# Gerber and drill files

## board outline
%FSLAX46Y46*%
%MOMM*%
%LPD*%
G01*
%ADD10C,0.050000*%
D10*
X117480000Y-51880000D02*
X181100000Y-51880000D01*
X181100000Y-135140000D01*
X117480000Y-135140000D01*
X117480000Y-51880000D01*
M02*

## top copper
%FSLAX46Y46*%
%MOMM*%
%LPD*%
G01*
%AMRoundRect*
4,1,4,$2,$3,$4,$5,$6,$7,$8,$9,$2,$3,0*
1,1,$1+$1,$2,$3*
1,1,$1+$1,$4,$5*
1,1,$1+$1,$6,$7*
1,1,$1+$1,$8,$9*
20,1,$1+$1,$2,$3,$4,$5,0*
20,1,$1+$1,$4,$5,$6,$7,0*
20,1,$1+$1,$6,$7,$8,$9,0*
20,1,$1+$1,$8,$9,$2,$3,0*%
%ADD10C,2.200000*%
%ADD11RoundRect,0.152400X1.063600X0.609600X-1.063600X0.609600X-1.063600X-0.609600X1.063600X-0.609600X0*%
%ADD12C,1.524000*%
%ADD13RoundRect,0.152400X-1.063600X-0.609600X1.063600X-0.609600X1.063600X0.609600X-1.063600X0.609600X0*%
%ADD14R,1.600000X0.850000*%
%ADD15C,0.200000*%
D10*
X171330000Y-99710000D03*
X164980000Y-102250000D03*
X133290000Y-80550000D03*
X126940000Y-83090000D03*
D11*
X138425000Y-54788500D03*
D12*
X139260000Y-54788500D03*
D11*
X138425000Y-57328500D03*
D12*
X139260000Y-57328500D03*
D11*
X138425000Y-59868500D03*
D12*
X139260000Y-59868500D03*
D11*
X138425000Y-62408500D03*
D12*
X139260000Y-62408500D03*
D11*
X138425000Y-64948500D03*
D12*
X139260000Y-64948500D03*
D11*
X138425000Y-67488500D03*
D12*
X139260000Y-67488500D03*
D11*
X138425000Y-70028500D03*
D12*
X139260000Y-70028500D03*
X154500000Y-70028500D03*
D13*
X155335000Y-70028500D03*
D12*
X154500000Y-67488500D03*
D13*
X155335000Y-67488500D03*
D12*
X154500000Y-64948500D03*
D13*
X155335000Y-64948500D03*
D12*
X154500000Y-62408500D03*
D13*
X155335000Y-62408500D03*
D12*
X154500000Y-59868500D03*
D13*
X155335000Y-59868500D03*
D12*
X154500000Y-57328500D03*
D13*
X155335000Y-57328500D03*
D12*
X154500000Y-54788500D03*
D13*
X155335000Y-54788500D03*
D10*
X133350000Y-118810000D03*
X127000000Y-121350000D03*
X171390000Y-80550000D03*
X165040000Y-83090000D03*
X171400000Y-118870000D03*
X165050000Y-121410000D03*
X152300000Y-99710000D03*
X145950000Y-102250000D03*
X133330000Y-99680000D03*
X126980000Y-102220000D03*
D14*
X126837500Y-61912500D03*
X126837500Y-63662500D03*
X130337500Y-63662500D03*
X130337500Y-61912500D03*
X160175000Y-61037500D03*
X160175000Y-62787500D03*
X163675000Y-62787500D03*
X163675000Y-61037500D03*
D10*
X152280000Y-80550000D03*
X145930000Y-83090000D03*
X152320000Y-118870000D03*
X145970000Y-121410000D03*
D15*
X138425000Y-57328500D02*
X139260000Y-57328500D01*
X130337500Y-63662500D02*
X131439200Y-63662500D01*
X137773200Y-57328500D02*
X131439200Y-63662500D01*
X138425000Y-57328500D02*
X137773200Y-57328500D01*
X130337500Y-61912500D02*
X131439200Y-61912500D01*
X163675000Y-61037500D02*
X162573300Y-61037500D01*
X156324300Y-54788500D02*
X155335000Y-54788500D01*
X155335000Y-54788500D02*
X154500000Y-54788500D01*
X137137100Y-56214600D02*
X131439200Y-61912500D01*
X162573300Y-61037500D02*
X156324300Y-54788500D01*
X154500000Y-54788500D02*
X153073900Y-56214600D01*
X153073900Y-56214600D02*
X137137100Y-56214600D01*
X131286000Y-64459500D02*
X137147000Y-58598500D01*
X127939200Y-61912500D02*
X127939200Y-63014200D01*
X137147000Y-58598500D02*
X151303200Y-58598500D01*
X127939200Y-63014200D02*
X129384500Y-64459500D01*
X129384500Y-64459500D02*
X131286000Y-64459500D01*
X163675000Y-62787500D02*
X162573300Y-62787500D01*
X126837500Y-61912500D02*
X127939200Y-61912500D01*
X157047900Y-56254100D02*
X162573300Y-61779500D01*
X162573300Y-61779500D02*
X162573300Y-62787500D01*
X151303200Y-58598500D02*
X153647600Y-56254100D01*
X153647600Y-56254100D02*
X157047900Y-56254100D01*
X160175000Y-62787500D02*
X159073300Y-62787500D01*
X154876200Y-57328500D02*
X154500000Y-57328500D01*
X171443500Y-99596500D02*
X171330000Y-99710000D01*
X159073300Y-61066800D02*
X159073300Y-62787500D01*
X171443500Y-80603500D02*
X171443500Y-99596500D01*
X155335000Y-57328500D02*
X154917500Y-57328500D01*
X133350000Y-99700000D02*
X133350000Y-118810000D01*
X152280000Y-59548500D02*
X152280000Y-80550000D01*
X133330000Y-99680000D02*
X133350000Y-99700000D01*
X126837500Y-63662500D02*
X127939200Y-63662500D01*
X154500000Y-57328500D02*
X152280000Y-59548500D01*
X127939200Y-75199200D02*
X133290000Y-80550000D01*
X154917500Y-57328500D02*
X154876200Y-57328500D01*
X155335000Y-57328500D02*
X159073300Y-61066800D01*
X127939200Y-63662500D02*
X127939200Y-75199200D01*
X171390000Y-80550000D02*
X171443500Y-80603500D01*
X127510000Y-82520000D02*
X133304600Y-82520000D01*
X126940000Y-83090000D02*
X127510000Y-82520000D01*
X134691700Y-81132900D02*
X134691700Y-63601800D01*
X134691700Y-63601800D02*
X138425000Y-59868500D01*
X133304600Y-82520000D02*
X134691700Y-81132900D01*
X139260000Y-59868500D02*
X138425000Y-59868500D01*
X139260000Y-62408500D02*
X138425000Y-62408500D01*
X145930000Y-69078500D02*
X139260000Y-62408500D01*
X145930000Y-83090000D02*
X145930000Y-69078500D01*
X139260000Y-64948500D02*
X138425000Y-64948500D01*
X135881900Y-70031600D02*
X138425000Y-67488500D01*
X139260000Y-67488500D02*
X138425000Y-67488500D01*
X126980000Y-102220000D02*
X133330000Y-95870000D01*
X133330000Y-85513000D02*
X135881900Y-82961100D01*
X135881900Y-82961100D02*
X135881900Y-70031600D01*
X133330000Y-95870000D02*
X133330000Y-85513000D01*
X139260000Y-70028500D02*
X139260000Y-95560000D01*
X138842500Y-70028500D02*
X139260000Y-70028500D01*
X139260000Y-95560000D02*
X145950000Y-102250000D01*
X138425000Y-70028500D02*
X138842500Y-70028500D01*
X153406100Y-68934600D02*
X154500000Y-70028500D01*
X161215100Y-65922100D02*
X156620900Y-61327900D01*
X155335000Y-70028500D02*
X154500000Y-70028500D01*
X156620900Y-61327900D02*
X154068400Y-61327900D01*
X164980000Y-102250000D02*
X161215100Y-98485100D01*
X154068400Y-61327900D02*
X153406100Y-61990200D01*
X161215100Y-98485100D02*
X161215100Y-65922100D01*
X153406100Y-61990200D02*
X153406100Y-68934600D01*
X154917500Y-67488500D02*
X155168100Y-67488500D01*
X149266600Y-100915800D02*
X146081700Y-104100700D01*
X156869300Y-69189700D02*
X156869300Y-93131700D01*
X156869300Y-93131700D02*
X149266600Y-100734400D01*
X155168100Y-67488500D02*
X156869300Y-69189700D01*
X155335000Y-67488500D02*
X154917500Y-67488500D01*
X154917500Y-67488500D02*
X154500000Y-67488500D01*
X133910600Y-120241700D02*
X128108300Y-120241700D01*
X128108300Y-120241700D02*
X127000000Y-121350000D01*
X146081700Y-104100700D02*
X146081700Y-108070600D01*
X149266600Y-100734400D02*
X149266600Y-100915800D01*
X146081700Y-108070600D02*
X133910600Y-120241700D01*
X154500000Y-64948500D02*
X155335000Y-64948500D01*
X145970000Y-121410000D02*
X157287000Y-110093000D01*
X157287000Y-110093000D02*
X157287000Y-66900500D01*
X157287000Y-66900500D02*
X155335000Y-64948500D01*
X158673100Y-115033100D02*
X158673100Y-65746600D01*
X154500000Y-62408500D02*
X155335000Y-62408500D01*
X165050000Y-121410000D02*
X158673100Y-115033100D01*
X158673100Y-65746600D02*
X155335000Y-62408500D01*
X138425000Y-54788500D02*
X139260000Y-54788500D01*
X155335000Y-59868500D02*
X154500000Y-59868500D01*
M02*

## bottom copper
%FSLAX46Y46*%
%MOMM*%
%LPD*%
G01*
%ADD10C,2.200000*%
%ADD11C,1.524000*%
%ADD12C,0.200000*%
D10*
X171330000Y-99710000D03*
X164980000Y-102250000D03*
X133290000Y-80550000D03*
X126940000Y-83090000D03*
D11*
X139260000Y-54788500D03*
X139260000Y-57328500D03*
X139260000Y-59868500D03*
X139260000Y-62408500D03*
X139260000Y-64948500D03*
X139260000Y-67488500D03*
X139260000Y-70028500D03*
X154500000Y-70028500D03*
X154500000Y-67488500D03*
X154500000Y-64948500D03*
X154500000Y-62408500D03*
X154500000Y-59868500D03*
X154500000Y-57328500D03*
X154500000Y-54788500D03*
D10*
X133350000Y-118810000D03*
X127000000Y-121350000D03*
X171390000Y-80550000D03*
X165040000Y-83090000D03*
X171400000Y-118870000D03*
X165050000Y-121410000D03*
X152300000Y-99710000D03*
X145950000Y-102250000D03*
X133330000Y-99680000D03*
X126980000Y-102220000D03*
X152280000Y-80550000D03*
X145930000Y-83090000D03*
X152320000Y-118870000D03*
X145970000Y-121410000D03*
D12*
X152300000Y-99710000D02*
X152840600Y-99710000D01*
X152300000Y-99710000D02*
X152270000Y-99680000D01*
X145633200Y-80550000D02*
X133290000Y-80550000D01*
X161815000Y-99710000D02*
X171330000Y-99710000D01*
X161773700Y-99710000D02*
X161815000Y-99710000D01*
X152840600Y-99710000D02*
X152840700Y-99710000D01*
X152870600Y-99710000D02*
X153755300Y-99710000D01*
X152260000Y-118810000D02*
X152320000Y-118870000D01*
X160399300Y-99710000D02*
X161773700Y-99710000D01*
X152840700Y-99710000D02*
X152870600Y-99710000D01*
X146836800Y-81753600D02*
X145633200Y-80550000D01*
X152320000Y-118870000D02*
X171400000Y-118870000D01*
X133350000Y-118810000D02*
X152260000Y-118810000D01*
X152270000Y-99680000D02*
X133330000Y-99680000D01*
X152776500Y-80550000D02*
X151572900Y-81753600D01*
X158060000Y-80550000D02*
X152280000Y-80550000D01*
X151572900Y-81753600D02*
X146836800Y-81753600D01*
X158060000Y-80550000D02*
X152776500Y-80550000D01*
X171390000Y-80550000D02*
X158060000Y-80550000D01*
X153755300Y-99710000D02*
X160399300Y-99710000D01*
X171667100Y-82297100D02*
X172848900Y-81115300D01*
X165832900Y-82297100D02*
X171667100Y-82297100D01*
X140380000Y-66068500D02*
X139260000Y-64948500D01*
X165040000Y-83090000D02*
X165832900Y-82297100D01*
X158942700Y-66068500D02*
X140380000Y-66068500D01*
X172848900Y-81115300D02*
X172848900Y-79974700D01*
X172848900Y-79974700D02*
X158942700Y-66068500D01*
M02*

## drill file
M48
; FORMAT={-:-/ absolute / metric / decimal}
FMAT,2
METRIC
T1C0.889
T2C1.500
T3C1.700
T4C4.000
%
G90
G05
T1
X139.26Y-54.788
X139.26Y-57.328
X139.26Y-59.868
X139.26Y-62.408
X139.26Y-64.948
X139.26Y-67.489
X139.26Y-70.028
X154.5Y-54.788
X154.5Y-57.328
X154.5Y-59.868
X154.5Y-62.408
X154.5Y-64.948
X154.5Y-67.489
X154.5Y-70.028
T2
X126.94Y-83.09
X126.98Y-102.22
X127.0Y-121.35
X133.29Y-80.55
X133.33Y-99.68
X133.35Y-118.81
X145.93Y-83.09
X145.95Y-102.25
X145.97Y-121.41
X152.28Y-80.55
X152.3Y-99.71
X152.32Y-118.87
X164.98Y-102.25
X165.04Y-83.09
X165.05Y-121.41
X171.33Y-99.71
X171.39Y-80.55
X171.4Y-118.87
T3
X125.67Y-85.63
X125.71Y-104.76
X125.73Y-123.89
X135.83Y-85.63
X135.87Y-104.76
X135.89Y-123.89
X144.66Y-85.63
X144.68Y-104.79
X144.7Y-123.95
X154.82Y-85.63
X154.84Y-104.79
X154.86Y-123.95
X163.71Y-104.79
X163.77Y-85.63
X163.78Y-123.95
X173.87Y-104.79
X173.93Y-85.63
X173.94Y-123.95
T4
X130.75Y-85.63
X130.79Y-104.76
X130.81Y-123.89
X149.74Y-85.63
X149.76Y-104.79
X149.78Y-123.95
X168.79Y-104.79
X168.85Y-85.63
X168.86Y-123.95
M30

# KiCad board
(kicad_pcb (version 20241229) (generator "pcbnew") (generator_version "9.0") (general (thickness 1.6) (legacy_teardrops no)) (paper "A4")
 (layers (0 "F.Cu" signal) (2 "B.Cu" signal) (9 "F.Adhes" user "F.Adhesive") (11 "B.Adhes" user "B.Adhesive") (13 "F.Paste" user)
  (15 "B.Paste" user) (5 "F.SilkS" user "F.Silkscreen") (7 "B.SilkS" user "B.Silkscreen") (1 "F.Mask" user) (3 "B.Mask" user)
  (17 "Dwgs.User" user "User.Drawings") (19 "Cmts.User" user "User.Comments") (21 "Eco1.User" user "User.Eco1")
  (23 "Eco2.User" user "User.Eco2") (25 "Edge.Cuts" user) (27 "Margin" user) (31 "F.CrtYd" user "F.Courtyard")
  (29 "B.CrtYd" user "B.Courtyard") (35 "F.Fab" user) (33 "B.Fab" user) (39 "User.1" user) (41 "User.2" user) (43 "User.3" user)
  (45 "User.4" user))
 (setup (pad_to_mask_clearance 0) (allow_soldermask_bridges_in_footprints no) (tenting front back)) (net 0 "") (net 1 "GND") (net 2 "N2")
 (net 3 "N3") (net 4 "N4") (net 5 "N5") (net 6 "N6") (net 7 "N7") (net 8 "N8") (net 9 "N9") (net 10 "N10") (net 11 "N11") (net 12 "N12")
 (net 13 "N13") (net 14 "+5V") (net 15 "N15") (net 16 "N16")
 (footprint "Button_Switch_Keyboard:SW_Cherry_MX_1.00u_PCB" (layer "F.Cu") (at 171.33 99.71)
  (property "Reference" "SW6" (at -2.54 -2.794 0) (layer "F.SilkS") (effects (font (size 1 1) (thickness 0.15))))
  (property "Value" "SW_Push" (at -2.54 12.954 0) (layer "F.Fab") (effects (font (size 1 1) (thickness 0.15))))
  (pad "" np_thru_hole circle (at -7.62 5.08) (size 1.7 1.7) (drill 1.7) (layers "*.Cu" "*.Mask"))
  (pad "" np_thru_hole circle (at -2.54 5.08) (size 4 4) (drill 4) (layers "*.Cu" "*.Mask"))
  (pad "" np_thru_hole circle (at 2.54 5.08) (size 1.7 1.7) (drill 1.7) (layers "*.Cu" "*.Mask"))
  (pad "1" thru_hole circle (at 0 0) (size 2.2 2.2) (drill 1.5) (layers "*.Cu" "*.Mask") (remove_unused_layers no) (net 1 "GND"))
  (pad "2" thru_hole circle (at -6.35 2.54) (size 2.2 2.2) (drill 1.5) (layers "*.Cu" "*.Mask") (remove_unused_layers no) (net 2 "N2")))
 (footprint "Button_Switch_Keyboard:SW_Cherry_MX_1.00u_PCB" (layer "F.Cu") (at 133.29 80.55)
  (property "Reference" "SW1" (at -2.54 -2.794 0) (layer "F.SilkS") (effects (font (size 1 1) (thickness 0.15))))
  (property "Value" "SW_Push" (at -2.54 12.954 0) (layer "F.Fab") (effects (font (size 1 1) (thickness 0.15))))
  (pad "" np_thru_hole circle (at -7.62 5.08) (size 1.7 1.7) (drill 1.7) (layers "*.Cu" "*.Mask"))
  (pad "" np_thru_hole circle (at -2.54 5.08) (size 4 4) (drill 4) (layers "*.Cu" "*.Mask"))
  (pad "" np_thru_hole circle (at 2.54 5.08) (size 1.7 1.7) (drill 1.7) (layers "*.Cu" "*.Mask"))
  (pad "1" thru_hole circle (at 0 0) (size 2.2 2.2) (drill 1.5) (layers "*.Cu" "*.Mask") (remove_unused_layers no) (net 1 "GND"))
  (pad "2" thru_hole circle (at -6.35 2.54) (size 2.2 2.2) (drill 1.5) (layers "*.Cu" "*.Mask") (remove_unused_layers no) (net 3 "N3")))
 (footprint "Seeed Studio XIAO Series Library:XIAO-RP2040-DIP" (layer "F.Cu") (at 146.88 62.4085)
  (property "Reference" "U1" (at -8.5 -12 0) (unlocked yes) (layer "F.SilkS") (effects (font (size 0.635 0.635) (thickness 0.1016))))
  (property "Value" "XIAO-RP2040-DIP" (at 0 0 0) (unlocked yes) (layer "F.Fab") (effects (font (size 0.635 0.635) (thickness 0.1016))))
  (pad "1" smd roundrect (at -8.455 -7.62 180) (size 2.432 1.524) (layers "F.Cu" "F.Mask") (roundrect_rratio 0.1) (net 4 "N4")
   (thermal_bridge_angle 45))
  (pad "1" thru_hole circle (at -7.62 -7.62 180) (size 1.524 1.524) (drill 0.889) (layers "*.Cu" "*.Mask") (remove_unused_layers no)
   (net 4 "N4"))
  (pad "2" smd roundrect (at -8.455 -5.08 180) (size 2.432 1.524) (layers "F.Cu" "F.Mask") (roundrect_rratio 0.1) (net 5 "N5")
   (thermal_bridge_angle 45))
  (pad "2" thru_hole circle (at -7.62 -5.08 180) (size 1.524 1.524) (drill 0.889) (layers "*.Cu" "*.Mask") (remove_unused_layers no)
   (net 5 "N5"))
  (pad "3" smd roundrect (at -8.455 -2.54 180) (size 2.432 1.524) (layers "F.Cu" "F.Mask") (roundrect_rratio 0.1) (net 3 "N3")
   (thermal_bridge_angle 45))
  (pad "3" thru_hole circle (at -7.62 -2.54 180) (size 1.524 1.524) (drill 0.889) (layers "*.Cu" "*.Mask") (remove_unused_layers no)
   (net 3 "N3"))
  (pad "4" smd roundrect (at -8.455 0 180) (size 2.432 1.524) (layers "F.Cu" "F.Mask") (roundrect_rratio 0.1) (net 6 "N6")
   (thermal_bridge_angle 45))
  (pad "4" thru_hole circle (at -7.62 0 180) (size 1.524 1.524) (drill 0.889) (layers "*.Cu" "*.Mask") (remove_unused_layers no)
   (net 6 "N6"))
  (pad "5" smd roundrect (at -8.455 2.54 180) (size 2.432 1.524) (layers "F.Cu" "F.Mask") (roundrect_rratio 0.1) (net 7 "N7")
   (thermal_bridge_angle 45))
  (pad "5" thru_hole circle (at -7.62 2.54 180) (size 1.524 1.524) (drill 0.889) (layers "*.Cu" "*.Mask") (remove_unused_layers no)
   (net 7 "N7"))
  (pad "6" smd roundrect (at -8.455 5.08 180) (size 2.432 1.524) (layers "F.Cu" "F.Mask") (roundrect_rratio 0.1) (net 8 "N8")
   (thermal_bridge_angle 45))
  (pad "6" thru_hole circle (at -7.62 5.08 180) (size 1.524 1.524) (drill 0.889) (layers "*.Cu" "*.Mask") (remove_unused_layers no)
   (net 8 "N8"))
  (pad "7" smd roundrect (at -8.455 7.62 180) (size 2.432 1.524) (layers "F.Cu" "F.Mask") (roundrect_rratio 0.1) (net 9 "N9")
   (thermal_bridge_angle 45))
  (pad "7" thru_hole circle (at -7.62 7.62 180) (size 1.524 1.524) (drill 0.889) (layers "*.Cu" "*.Mask") (remove_unused_layers no)
   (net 9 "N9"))
  (pad "8" thru_hole circle (at 7.62 7.62) (size 1.524 1.524) (drill 0.889) (layers "*.Cu" "*.Mask") (remove_unused_layers no) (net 2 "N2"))
  (pad "8" smd roundrect (at 8.455 7.62) (size 2.432 1.524) (layers "F.Cu" "F.Mask") (roundrect_rratio 0.1) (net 2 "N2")
   (thermal_bridge_angle 45))
  (pad "9" thru_hole circle (at 7.62 5.08) (size 1.524 1.524) (drill 0.889) (layers "*.Cu" "*.Mask") (remove_unused_layers no)
   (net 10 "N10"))
  (pad "9" smd roundrect (at 8.455 5.08) (size 2.432 1.524) (layers "F.Cu" "F.Mask") (roundrect_rratio 0.1) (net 10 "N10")
   (thermal_bridge_angle 45))
  (pad "10" thru_hole circle (at 7.62 2.54) (size 1.524 1.524) (drill 0.889) (layers "*.Cu" "*.Mask") (remove_unused_layers no)
   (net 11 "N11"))
  (pad "10" smd roundrect (at 8.455 2.54) (size 2.432 1.524) (layers "F.Cu" "F.Mask") (roundrect_rratio 0.1) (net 11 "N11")
   (thermal_bridge_angle 45))
  (pad "11" thru_hole circle (at 7.62 0) (size 1.524 1.524) (drill 0.889) (layers "*.Cu" "*.Mask") (remove_unused_layers no) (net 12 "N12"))
  (pad "11" smd roundrect (at 8.455 0) (size 2.432 1.524) (layers "F.Cu" "F.Mask") (roundrect_rratio 0.1) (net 12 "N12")
   (thermal_bridge_angle 45))
  (pad "12" thru_hole circle (at 7.62 -2.54) (size 1.524 1.524) (drill 0.889) (layers "*.Cu" "*.Mask") (remove_unused_layers no)
   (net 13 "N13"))
  (pad "12" smd roundrect (at 8.455 -2.54) (size 2.432 1.524) (layers "F.Cu" "F.Mask") (roundrect_rratio 0.1) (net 13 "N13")
   (thermal_bridge_angle 45))
  (pad "13" thru_hole circle (at 7.62 -5.08) (size 1.524 1.524) (drill 0.889) (layers "*.Cu" "*.Mask") (remove_unused_layers no)
   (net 1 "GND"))
  (pad "13" smd roundrect (at 8.455 -5.08) (size 2.432 1.524) (layers "F.Cu" "F.Mask") (roundrect_rratio 0.1) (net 1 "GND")
   (thermal_bridge_angle 45))
  (pad "14" thru_hole circle (at 7.62 -7.62) (size 1.524 1.524) (drill 0.889) (layers "*.Cu" "*.Mask") (remove_unused_layers no)
   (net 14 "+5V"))
  (pad "14" smd roundrect (at 8.455 -7.62) (size 2.432 1.524) (layers "F.Cu" "F.Mask") (roundrect_rratio 0.1) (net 14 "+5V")
   (thermal_bridge_angle 45)))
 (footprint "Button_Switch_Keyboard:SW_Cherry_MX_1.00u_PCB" (layer "F.Cu") (at 133.35 118.81)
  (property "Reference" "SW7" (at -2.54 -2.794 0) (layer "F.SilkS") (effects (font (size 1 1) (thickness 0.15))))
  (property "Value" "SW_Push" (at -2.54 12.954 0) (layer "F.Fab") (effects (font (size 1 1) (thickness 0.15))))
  (pad "" np_thru_hole circle (at -7.62 5.08) (size 1.7 1.7) (drill 1.7) (layers "*.Cu" "*.Mask"))
  (pad "" np_thru_hole circle (at -2.54 5.08) (size 4 4) (drill 4) (layers "*.Cu" "*.Mask"))
  (pad "" np_thru_hole circle (at 2.54 5.08) (size 1.7 1.7) (drill 1.7) (layers "*.Cu" "*.Mask"))
  (pad "1" thru_hole circle (at 0 0) (size 2.2 2.2) (drill 1.5) (layers "*.Cu" "*.Mask") (remove_unused_layers no) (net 1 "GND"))
  (pad "2" thru_hole circle (at -6.35 2.54) (size 2.2 2.2) (drill 1.5) (layers "*.Cu" "*.Mask") (remove_unused_layers no) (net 10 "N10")))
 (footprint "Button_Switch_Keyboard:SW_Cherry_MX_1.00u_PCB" (layer "F.Cu") (at 171.39 80.55)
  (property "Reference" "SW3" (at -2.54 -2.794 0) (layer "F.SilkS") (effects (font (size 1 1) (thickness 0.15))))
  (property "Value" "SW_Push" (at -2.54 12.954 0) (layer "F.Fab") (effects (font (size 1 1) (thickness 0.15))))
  (pad "" np_thru_hole circle (at -7.62 5.08) (size 1.7 1.7) (drill 1.7) (layers "*.Cu" "*.Mask"))
  (pad "" np_thru_hole circle (at -2.54 5.08) (size 4 4) (drill 4) (layers "*.Cu" "*.Mask"))
  (pad "" np_thru_hole circle (at 2.54 5.08) (size 1.7 1.7) (drill 1.7) (layers "*.Cu" "*.Mask"))
  (pad "1" thru_hole circle (at 0 0) (size 2.2 2.2) (drill 1.5) (layers "*.Cu" "*.Mask") (remove_unused_layers no) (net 1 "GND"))
  (pad "2" thru_hole circle (at -6.35 2.54) (size 2.2 2.2) (drill 1.5) (layers "*.Cu" "*.Mask") (remove_unused_layers no) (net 7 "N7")))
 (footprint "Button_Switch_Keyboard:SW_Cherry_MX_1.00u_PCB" (layer "F.Cu") (at 171.4 118.87)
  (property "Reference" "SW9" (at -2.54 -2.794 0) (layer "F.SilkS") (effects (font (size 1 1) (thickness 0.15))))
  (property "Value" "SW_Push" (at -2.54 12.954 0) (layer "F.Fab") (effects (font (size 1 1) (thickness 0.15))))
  (pad "" np_thru_hole circle (at -7.62 5.08) (size 1.7 1.7) (drill 1.7) (layers "*.Cu" "*.Mask"))
  (pad "" np_thru_hole circle (at -2.54 5.08) (size 4 4) (drill 4) (layers "*.Cu" "*.Mask"))
  (pad "" np_thru_hole circle (at 2.54 5.08) (size 1.7 1.7) (drill 1.7) (layers "*.Cu" "*.Mask"))
  (pad "1" thru_hole circle (at 0 0) (size 2.2 2.2) (drill 1.5) (layers "*.Cu" "*.Mask") (remove_unused_layers no) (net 1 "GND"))
  (pad "2" thru_hole circle (at -6.35 2.54) (size 2.2 2.2) (drill 1.5) (layers "*.Cu" "*.Mask") (remove_unused_layers no) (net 12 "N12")))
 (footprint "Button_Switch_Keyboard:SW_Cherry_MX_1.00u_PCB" (layer "F.Cu") (at 152.3 99.71)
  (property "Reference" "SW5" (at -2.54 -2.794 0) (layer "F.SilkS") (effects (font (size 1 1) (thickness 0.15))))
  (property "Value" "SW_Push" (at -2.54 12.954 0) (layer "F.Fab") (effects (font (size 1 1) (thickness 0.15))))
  (pad "" np_thru_hole circle (at -7.62 5.08) (size 1.7 1.7) (drill 1.7) (layers "*.Cu" "*.Mask"))
  (pad "" np_thru_hole circle (at -2.54 5.08) (size 4 4) (drill 4) (layers "*.Cu" "*.Mask"))
  (pad "" np_thru_hole circle (at 2.54 5.08) (size 1.7 1.7) (drill 1.7) (layers "*.Cu" "*.Mask"))
  (pad "1" thru_hole circle (at 0 0) (size 2.2 2.2) (drill 1.5) (layers "*.Cu" "*.Mask") (remove_unused_layers no) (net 1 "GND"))
  (pad "2" thru_hole circle (at -6.35 2.54) (size 2.2 2.2) (drill 1.5) (layers "*.Cu" "*.Mask") (remove_unused_layers no) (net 9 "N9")))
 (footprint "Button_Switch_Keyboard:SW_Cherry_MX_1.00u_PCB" (layer "F.Cu") (at 133.33 99.68)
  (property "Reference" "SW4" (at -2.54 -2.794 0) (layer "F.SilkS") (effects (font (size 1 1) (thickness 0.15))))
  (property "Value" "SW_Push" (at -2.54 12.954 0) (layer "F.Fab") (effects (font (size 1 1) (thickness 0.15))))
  (pad "" np_thru_hole circle (at -7.62 5.08) (size 1.7 1.7) (drill 1.7) (layers "*.Cu" "*.Mask"))
  (pad "" np_thru_hole circle (at -2.54 5.08) (size 4 4) (drill 4) (layers "*.Cu" "*.Mask"))
  (pad "" np_thru_hole circle (at 2.54 5.08) (size 1.7 1.7) (drill 1.7) (layers "*.Cu" "*.Mask"))
  (pad "1" thru_hole circle (at 0 0) (size 2.2 2.2) (drill 1.5) (layers "*.Cu" "*.Mask") (remove_unused_layers no) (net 1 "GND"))
  (pad "2" thru_hole circle (at -6.35 2.54) (size 2.2 2.2) (drill 1.5) (layers "*.Cu" "*.Mask") (remove_unused_layers no) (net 8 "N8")))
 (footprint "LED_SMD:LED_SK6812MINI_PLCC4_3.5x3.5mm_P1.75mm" (layer "F.Cu") (at 128.5875 62.7875)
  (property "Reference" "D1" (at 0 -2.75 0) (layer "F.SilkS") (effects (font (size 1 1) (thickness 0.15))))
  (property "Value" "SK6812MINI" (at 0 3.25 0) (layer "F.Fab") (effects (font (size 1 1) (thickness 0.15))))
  (pad "1" smd rect (at -1.75 -0.875) (size 1.6 0.85) (layers "F.Cu" "F.Mask" "F.Paste") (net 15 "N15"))
  (pad "2" smd rect (at -1.75 0.875) (size 1.6 0.85) (layers "F.Cu" "F.Mask" "F.Paste") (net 1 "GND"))
  (pad "3" smd rect (at 1.75 0.875) (size 1.6 0.85) (layers "F.Cu" "F.Mask" "F.Paste") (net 5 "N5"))
  (pad "4" smd rect (at 1.75 -0.875) (size 1.6 0.85) (layers "F.Cu" "F.Mask" "F.Paste") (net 14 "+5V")))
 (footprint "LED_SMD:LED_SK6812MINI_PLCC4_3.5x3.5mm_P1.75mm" (layer "F.Cu") (at 161.925 61.9125)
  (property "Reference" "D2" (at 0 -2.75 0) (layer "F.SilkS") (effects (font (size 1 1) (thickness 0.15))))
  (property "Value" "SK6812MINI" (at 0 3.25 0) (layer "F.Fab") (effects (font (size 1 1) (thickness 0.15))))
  (pad "1" smd rect (at -1.75 -0.875) (size 1.6 0.85) (layers "F.Cu" "F.Mask" "F.Paste") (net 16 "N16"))
  (pad "2" smd rect (at -1.75 0.875) (size 1.6 0.85) (layers "F.Cu" "F.Mask" "F.Paste") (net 1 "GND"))
  (pad "3" smd rect (at 1.75 0.875) (size 1.6 0.85) (layers "F.Cu" "F.Mask" "F.Paste") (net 15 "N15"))
  (pad "4" smd rect (at 1.75 -0.875) (size 1.6 0.85) (layers "F.Cu" "F.Mask" "F.Paste") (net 14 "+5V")))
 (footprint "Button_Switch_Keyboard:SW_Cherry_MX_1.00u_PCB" (layer "F.Cu") (at 152.28 80.55)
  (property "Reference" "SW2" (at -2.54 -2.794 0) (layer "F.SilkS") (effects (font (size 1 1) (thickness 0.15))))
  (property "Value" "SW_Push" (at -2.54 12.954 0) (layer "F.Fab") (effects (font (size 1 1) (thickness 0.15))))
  (pad "" np_thru_hole circle (at -7.62 5.08) (size 1.7 1.7) (drill 1.7) (layers "*.Cu" "*.Mask"))
  (pad "" np_thru_hole circle (at -2.54 5.08) (size 4 4) (drill 4) (layers "*.Cu" "*.Mask"))
  (pad "" np_thru_hole circle (at 2.54 5.08) (size 1.7 1.7) (drill 1.7) (layers "*.Cu" "*.Mask"))
  (pad "1" thru_hole circle (at 0 0) (size 2.2 2.2) (drill 1.5) (layers "*.Cu" "*.Mask") (remove_unused_layers no) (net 1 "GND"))
  (pad "2" thru_hole circle (at -6.35 2.54) (size 2.2 2.2) (drill 1.5) (layers "*.Cu" "*.Mask") (remove_unused_layers no) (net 6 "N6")))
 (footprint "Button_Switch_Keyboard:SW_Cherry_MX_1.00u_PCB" (layer "F.Cu") (at 152.32 118.87)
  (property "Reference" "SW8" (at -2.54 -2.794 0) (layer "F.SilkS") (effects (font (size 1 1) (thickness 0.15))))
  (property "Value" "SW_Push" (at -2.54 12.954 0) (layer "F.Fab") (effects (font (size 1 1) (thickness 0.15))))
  (pad "" np_thru_hole circle (at -7.62 5.08) (size 1.7 1.7) (drill 1.7) (layers "*.Cu" "*.Mask"))
  (pad "" np_thru_hole circle (at -2.54 5.08) (size 4 4) (drill 4) (layers "*.Cu" "*.Mask"))
  (pad "" np_thru_hole circle (at 2.54 5.08) (size 1.7 1.7) (drill 1.7) (layers "*.Cu" "*.Mask"))
  (pad "1" thru_hole circle (at 0 0) (size 2.2 2.2) (drill 1.5) (layers "*.Cu" "*.Mask") (remove_unused_layers no) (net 1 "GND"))
  (pad "2" thru_hole circle (at -6.35 2.54) (size 2.2 2.2) (drill 1.5) (layers "*.Cu" "*.Mask") (remove_unused_layers no) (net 11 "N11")))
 (gr_rect (start 117.48 51.88) (end 181.1 135.14) (stroke (width 0.05) (type default)) (fill no) (layer "Edge.Cuts"))
 (segment (start 138.425 57.3285) (end 139.26 57.3285) (width 0.2) (layer "F.Cu") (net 5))
 (segment (start 130.3375 63.6625) (end 131.4392 63.6625) (width 0.2) (layer "F.Cu") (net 5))
 (segment (start 137.7732 57.3285) (end 131.4392 63.6625) (width 0.2) (layer "F.Cu") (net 5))
 (segment (start 138.425 57.3285) (end 137.7732 57.3285) (width 0.2) (layer "F.Cu") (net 5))
 (segment (start 130.3375 61.9125) (end 131.4392 61.9125) (width 0.2) (layer "F.Cu") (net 14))
 (segment (start 163.675 61.0375) (end 162.5733 61.0375) (width 0.2) (layer "F.Cu") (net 14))
 (segment (start 156.3243 54.7885) (end 155.335 54.7885) (width 0.2) (layer "F.Cu") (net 14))
 (segment (start 155.335 54.7885) (end 154.5 54.7885) (width 0.2) (layer "F.Cu") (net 14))
 (segment (start 137.1371 56.2146) (end 131.4392 61.9125) (width 0.2) (layer "F.Cu") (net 14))
 (segment (start 162.5733 61.0375) (end 156.3243 54.7885) (width 0.2) (layer "F.Cu") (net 14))
 (segment (start 154.5 54.7885) (end 153.0739 56.2146) (width 0.2) (layer "F.Cu") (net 14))
 (segment (start 153.0739 56.2146) (end 137.1371 56.2146) (width 0.2) (layer "F.Cu") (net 14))
 (segment (start 131.286 64.4595) (end 137.147 58.5985) (width 0.2) (layer "F.Cu") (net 15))
 (segment (start 127.9392 61.9125) (end 127.9392 63.0142) (width 0.2) (layer "F.Cu") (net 15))
 (segment (start 137.147 58.5985) (end 151.3032 58.5985) (width 0.2) (layer "F.Cu") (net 15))
 (segment (start 127.9392 63.0142) (end 129.3845 64.4595) (width 0.2) (layer "F.Cu") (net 15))
 (segment (start 129.3845 64.4595) (end 131.286 64.4595) (width 0.2) (layer "F.Cu") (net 15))
 (segment (start 163.675 62.7875) (end 162.5733 62.7875) (width 0.2) (layer "F.Cu") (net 15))
 (segment (start 126.8375 61.9125) (end 127.9392 61.9125) (width 0.2) (layer "F.Cu") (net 15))
 (segment (start 157.0479 56.2541) (end 162.5733 61.7795) (width 0.2) (layer "F.Cu") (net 15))
 (segment (start 162.5733 61.7795) (end 162.5733 62.7875) (width 0.2) (layer "F.Cu") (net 15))
 (segment (start 151.3032 58.5985) (end 153.6476 56.2541) (width 0.2) (layer "F.Cu") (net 15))
 (segment (start 153.6476 56.2541) (end 157.0479 56.2541) (width 0.2) (layer "F.Cu") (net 15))
 (segment (start 160.175 62.7875) (end 159.0733 62.7875) (width 0.2) (layer "F.Cu") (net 1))
 (segment (start 154.8762 57.3285) (end 154.5 57.3285) (width 0.2) (layer "F.Cu") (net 1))
 (segment (start 171.4435 99.5965) (end 171.33 99.71) (width 0.2) (layer "F.Cu") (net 1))
 (segment (start 159.0733 61.0668) (end 159.0733 62.7875) (width 0.2) (layer "F.Cu") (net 1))
 (segment (start 171.4435 80.6035) (end 171.4435 99.5965) (width 0.2) (layer "F.Cu") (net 1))
 (segment (start 155.335 57.3285) (end 154.9175 57.3285) (width 0.2) (layer "F.Cu") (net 1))
 (segment (start 133.35 99.7) (end 133.35 118.81) (width 0.2) (layer "F.Cu") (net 1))
 (segment (start 152.28 59.5485) (end 152.28 80.55) (width 0.2) (layer "F.Cu") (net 1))
 (segment (start 133.33 99.68) (end 133.35 99.7) (width 0.2) (layer "F.Cu") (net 1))
 (segment (start 126.8375 63.6625) (end 127.9392 63.6625) (width 0.2) (layer "F.Cu") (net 1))
 (segment (start 154.5 57.3285) (end 152.28 59.5485) (width 0.2) (layer "F.Cu") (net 1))
 (segment (start 127.9392 75.1992) (end 133.29 80.55) (width 0.2) (layer "F.Cu") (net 1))
 (segment (start 154.9175 57.3285) (end 154.8762 57.3285) (width 0.2) (layer "F.Cu") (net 1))
 (segment (start 155.335 57.3285) (end 159.0733 61.0668) (width 0.2) (layer "F.Cu") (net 1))
 (segment (start 127.9392 63.6625) (end 127.9392 75.1992) (width 0.2) (layer "F.Cu") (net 1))
 (segment (start 171.39 80.55) (end 171.4435 80.6035) (width 0.2) (layer "F.Cu") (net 1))
 (segment (start 152.3 99.71) (end 152.8406 99.71) (width 0.2) (layer "B.Cu") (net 1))
 (segment (start 152.3 99.71) (end 152.27 99.68) (width 0.2) (layer "B.Cu") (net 1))
 (segment (start 145.6332 80.55) (end 133.29 80.55) (width 0.2) (layer "B.Cu") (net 1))
 (segment (start 161.815 99.71) (end 171.33 99.71) (width 0.2) (layer "B.Cu") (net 1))
 (segment (start 161.7737 99.71) (end 161.815 99.71) (width 0.2) (layer "B.Cu") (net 1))
 (segment (start 152.8406 99.71) (end 152.8407 99.71) (width 0.2) (layer "B.Cu") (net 1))
 (segment (start 152.8706 99.71) (end 153.7553 99.71) (width 0.2) (layer "B.Cu") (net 1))
 (segment (start 152.26 118.81) (end 152.32 118.87) (width 0.2) (layer "B.Cu") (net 1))
 (segment (start 160.3993 99.71) (end 161.7737 99.71) (width 0.2) (layer "B.Cu") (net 1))
 (segment (start 152.8407 99.71) (end 152.8706 99.71) (width 0.2) (layer "B.Cu") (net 1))
 (segment (start 146.8368 81.7536) (end 145.6332 80.55) (width 0.2) (layer "B.Cu") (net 1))
 (segment (start 152.32 118.87) (end 171.4 118.87) (width 0.2) (layer "B.Cu") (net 1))
 (segment (start 133.35 118.81) (end 152.26 118.81) (width 0.2) (layer "B.Cu") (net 1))
 (segment (start 152.27 99.68) (end 133.33 99.68) (width 0.2) (layer "B.Cu") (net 1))
 (segment (start 152.7765 80.55) (end 151.5729 81.7536) (width 0.2) (layer "B.Cu") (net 1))
 (segment (start 158.06 80.55) (end 152.28 80.55) (width 0.2) (layer "B.Cu") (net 1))
 (segment (start 151.5729 81.7536) (end 146.8368 81.7536) (width 0.2) (layer "B.Cu") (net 1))
 (segment (start 158.06 80.55) (end 152.7765 80.55) (width 0.2) (layer "B.Cu") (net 1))
 (segment (start 171.39 80.55) (end 158.06 80.55) (width 0.2) (layer "B.Cu") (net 1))
 (segment (start 153.7553 99.71) (end 160.3993 99.71) (width 0.2) (layer "B.Cu") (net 1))
 (segment (start 127.51 82.52) (end 133.3046 82.52) (width 0.2) (layer "F.Cu") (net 3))
 (segment (start 126.94 83.09) (end 127.51 82.52) (width 0.2) (layer "F.Cu") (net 3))
 (segment (start 134.6917 81.1329) (end 134.6917 63.6018) (width 0.2) (layer "F.Cu") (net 3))
 (segment (start 134.6917 63.6018) (end 138.425 59.8685) (width 0.2) (layer "F.Cu") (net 3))
 (segment (start 133.3046 82.52) (end 134.6917 81.1329) (width 0.2) (layer "F.Cu") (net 3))
 (segment (start 139.26 59.8685) (end 138.425 59.8685) (width 0.2) (layer "F.Cu") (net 3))
 (segment (start 139.26 62.4085) (end 138.425 62.4085) (width 0.2) (layer "F.Cu") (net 6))
 (segment (start 145.93 69.0785) (end 139.26 62.4085) (width 0.2) (layer "F.Cu") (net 6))
 (segment (start 145.93 83.09) (end 145.93 69.0785) (width 0.2) (layer "F.Cu") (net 6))
 (segment (start 139.26 64.9485) (end 138.425 64.9485) (width 0.2) (layer "F.Cu") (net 7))
 (segment (start 171.6671 82.2971) (end 172.8489 81.1153) (width 0.2) (layer "B.Cu") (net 7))
 (segment (start 165.8329 82.2971) (end 171.6671 82.2971) (width 0.2) (layer "B.Cu") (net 7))
 (segment (start 140.38 66.0685) (end 139.26 64.9485) (width 0.2) (layer "B.Cu") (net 7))
 (segment (start 165.04 83.09) (end 165.8329 82.2971) (width 0.2) (layer "B.Cu") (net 7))
 (segment (start 158.9427 66.0685) (end 140.38 66.0685) (width 0.2) (layer "B.Cu") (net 7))
 (segment (start 172.8489 81.1153) (end 172.8489 79.9747) (width 0.2) (layer "B.Cu") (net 7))
 (segment (start 172.8489 79.9747) (end 158.9427 66.0685) (width 0.2) (layer "B.Cu") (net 7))
 (segment (start 135.8819 70.0316) (end 138.425 67.4885) (width 0.2) (layer "F.Cu") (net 8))
 (segment (start 139.26 67.4885) (end 138.425 67.4885) (width 0.2) (layer "F.Cu") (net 8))
 (segment (start 126.98 102.22) (end 133.33 95.87) (width 0.2) (layer "F.Cu") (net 8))
 (segment (start 133.33 85.513) (end 135.8819 82.9611) (width 0.2) (layer "F.Cu") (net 8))
 (segment (start 135.8819 82.9611) (end 135.8819 70.0316) (width 0.2) (layer "F.Cu") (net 8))
 (segment (start 133.33 95.87) (end 133.33 85.513) (width 0.2) (layer "F.Cu") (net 8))
 (segment (start 139.26 70.0285) (end 139.26 95.56) (width 0.2) (layer "F.Cu") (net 9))
 (segment (start 138.8425 70.0285) (end 139.26 70.0285) (width 0.2) (layer "F.Cu") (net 9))
 (segment (start 139.26 95.56) (end 145.95 102.25) (width 0.2) (layer "F.Cu") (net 9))
 (segment (start 138.425 70.0285) (end 138.8425 70.0285) (width 0.2) (layer "F.Cu") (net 9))
 (segment (start 153.4061 68.9346) (end 154.5 70.0285) (width 0.2) (layer "F.Cu") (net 2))
 (segment (start 161.2151 65.9221) (end 156.6209 61.3279) (width 0.2) (layer "F.Cu") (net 2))
 (segment (start 155.335 70.0285) (end 154.5 70.0285) (width 0.2) (layer "F.Cu") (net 2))
 (segment (start 156.6209 61.3279) (end 154.0684 61.3279) (width 0.2) (layer "F.Cu") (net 2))
 (segment (start 164.98 102.25) (end 161.2151 98.4851) (width 0.2) (layer "F.Cu") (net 2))
 (segment (start 154.0684 61.3279) (end 153.4061 61.9902) (width 0.2) (layer "F.Cu") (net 2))
 (segment (start 161.2151 98.4851) (end 161.2151 65.9221) (width 0.2) (layer "F.Cu") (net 2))
 (segment (start 153.4061 61.9902) (end 153.4061 68.9346) (width 0.2) (layer "F.Cu") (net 2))
 (segment (start 154.9175 67.4885) (end 155.1681 67.4885) (width 0.2) (layer "F.Cu") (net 10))
 (segment (start 149.2666 100.9158) (end 146.0817 104.1007) (width 0.2) (layer "F.Cu") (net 10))
 (segment (start 156.8693 69.1897) (end 156.8693 93.1317) (width 0.2) (layer "F.Cu") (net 10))
 (segment (start 156.8693 93.1317) (end 149.2666 100.7344) (width 0.2) (layer "F.Cu") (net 10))
 (segment (start 155.1681 67.4885) (end 156.8693 69.1897) (width 0.2) (layer "F.Cu") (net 10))
 (segment (start 155.335 67.4885) (end 154.9175 67.4885) (width 0.2) (layer "F.Cu") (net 10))
 (segment (start 154.9175 67.4885) (end 154.5 67.4885) (width 0.2) (layer "F.Cu") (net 10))
 (segment (start 133.9106 120.2417) (end 128.1083 120.2417) (width 0.2) (layer "F.Cu") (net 10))
 (segment (start 128.1083 120.2417) (end 127 121.35) (width 0.2) (layer "F.Cu") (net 10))
 (segment (start 146.0817 104.1007) (end 146.0817 108.0706) (width 0.2) (layer "F.Cu") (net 10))
 (segment (start 149.2666 100.7344) (end 149.2666 100.9158) (width 0.2) (layer "F.Cu") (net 10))
 (segment (start 146.0817 108.0706) (end 133.9106 120.2417) (width 0.2) (layer "F.Cu") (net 10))
 (segment (start 154.5 64.9485) (end 155.335 64.9485) (width 0.2) (layer "F.Cu") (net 11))
 (segment (start 145.97 121.41) (end 157.287 110.093) (width 0.2) (layer "F.Cu") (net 11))
 (segment (start 157.287 110.093) (end 157.287 66.9005) (width 0.2) (layer "F.Cu") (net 11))
 (segment (start 157.287 66.9005) (end 155.335 64.9485) (width 0.2) (layer "F.Cu") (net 11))
 (segment (start 158.6731 115.0331) (end 158.6731 65.7466) (width 0.2) (layer "F.Cu") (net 12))
 (segment (start 154.5 62.4085) (end 155.335 62.4085) (width 0.2) (layer "F.Cu") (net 12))
 (segment (start 165.05 121.41) (end 158.6731 115.0331) (width 0.2) (layer "F.Cu") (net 12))
 (segment (start 158.6731 65.7466) (end 155.335 62.4085) (width 0.2) (layer "F.Cu") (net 12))
 (segment (start 138.425 54.7885) (end 139.26 54.7885) (width 0.2) (layer "F.Cu") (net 4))
 (segment (start 155.335 59.8685) (end 154.5 59.8685) (width 0.2) (layer "F.Cu") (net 13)))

